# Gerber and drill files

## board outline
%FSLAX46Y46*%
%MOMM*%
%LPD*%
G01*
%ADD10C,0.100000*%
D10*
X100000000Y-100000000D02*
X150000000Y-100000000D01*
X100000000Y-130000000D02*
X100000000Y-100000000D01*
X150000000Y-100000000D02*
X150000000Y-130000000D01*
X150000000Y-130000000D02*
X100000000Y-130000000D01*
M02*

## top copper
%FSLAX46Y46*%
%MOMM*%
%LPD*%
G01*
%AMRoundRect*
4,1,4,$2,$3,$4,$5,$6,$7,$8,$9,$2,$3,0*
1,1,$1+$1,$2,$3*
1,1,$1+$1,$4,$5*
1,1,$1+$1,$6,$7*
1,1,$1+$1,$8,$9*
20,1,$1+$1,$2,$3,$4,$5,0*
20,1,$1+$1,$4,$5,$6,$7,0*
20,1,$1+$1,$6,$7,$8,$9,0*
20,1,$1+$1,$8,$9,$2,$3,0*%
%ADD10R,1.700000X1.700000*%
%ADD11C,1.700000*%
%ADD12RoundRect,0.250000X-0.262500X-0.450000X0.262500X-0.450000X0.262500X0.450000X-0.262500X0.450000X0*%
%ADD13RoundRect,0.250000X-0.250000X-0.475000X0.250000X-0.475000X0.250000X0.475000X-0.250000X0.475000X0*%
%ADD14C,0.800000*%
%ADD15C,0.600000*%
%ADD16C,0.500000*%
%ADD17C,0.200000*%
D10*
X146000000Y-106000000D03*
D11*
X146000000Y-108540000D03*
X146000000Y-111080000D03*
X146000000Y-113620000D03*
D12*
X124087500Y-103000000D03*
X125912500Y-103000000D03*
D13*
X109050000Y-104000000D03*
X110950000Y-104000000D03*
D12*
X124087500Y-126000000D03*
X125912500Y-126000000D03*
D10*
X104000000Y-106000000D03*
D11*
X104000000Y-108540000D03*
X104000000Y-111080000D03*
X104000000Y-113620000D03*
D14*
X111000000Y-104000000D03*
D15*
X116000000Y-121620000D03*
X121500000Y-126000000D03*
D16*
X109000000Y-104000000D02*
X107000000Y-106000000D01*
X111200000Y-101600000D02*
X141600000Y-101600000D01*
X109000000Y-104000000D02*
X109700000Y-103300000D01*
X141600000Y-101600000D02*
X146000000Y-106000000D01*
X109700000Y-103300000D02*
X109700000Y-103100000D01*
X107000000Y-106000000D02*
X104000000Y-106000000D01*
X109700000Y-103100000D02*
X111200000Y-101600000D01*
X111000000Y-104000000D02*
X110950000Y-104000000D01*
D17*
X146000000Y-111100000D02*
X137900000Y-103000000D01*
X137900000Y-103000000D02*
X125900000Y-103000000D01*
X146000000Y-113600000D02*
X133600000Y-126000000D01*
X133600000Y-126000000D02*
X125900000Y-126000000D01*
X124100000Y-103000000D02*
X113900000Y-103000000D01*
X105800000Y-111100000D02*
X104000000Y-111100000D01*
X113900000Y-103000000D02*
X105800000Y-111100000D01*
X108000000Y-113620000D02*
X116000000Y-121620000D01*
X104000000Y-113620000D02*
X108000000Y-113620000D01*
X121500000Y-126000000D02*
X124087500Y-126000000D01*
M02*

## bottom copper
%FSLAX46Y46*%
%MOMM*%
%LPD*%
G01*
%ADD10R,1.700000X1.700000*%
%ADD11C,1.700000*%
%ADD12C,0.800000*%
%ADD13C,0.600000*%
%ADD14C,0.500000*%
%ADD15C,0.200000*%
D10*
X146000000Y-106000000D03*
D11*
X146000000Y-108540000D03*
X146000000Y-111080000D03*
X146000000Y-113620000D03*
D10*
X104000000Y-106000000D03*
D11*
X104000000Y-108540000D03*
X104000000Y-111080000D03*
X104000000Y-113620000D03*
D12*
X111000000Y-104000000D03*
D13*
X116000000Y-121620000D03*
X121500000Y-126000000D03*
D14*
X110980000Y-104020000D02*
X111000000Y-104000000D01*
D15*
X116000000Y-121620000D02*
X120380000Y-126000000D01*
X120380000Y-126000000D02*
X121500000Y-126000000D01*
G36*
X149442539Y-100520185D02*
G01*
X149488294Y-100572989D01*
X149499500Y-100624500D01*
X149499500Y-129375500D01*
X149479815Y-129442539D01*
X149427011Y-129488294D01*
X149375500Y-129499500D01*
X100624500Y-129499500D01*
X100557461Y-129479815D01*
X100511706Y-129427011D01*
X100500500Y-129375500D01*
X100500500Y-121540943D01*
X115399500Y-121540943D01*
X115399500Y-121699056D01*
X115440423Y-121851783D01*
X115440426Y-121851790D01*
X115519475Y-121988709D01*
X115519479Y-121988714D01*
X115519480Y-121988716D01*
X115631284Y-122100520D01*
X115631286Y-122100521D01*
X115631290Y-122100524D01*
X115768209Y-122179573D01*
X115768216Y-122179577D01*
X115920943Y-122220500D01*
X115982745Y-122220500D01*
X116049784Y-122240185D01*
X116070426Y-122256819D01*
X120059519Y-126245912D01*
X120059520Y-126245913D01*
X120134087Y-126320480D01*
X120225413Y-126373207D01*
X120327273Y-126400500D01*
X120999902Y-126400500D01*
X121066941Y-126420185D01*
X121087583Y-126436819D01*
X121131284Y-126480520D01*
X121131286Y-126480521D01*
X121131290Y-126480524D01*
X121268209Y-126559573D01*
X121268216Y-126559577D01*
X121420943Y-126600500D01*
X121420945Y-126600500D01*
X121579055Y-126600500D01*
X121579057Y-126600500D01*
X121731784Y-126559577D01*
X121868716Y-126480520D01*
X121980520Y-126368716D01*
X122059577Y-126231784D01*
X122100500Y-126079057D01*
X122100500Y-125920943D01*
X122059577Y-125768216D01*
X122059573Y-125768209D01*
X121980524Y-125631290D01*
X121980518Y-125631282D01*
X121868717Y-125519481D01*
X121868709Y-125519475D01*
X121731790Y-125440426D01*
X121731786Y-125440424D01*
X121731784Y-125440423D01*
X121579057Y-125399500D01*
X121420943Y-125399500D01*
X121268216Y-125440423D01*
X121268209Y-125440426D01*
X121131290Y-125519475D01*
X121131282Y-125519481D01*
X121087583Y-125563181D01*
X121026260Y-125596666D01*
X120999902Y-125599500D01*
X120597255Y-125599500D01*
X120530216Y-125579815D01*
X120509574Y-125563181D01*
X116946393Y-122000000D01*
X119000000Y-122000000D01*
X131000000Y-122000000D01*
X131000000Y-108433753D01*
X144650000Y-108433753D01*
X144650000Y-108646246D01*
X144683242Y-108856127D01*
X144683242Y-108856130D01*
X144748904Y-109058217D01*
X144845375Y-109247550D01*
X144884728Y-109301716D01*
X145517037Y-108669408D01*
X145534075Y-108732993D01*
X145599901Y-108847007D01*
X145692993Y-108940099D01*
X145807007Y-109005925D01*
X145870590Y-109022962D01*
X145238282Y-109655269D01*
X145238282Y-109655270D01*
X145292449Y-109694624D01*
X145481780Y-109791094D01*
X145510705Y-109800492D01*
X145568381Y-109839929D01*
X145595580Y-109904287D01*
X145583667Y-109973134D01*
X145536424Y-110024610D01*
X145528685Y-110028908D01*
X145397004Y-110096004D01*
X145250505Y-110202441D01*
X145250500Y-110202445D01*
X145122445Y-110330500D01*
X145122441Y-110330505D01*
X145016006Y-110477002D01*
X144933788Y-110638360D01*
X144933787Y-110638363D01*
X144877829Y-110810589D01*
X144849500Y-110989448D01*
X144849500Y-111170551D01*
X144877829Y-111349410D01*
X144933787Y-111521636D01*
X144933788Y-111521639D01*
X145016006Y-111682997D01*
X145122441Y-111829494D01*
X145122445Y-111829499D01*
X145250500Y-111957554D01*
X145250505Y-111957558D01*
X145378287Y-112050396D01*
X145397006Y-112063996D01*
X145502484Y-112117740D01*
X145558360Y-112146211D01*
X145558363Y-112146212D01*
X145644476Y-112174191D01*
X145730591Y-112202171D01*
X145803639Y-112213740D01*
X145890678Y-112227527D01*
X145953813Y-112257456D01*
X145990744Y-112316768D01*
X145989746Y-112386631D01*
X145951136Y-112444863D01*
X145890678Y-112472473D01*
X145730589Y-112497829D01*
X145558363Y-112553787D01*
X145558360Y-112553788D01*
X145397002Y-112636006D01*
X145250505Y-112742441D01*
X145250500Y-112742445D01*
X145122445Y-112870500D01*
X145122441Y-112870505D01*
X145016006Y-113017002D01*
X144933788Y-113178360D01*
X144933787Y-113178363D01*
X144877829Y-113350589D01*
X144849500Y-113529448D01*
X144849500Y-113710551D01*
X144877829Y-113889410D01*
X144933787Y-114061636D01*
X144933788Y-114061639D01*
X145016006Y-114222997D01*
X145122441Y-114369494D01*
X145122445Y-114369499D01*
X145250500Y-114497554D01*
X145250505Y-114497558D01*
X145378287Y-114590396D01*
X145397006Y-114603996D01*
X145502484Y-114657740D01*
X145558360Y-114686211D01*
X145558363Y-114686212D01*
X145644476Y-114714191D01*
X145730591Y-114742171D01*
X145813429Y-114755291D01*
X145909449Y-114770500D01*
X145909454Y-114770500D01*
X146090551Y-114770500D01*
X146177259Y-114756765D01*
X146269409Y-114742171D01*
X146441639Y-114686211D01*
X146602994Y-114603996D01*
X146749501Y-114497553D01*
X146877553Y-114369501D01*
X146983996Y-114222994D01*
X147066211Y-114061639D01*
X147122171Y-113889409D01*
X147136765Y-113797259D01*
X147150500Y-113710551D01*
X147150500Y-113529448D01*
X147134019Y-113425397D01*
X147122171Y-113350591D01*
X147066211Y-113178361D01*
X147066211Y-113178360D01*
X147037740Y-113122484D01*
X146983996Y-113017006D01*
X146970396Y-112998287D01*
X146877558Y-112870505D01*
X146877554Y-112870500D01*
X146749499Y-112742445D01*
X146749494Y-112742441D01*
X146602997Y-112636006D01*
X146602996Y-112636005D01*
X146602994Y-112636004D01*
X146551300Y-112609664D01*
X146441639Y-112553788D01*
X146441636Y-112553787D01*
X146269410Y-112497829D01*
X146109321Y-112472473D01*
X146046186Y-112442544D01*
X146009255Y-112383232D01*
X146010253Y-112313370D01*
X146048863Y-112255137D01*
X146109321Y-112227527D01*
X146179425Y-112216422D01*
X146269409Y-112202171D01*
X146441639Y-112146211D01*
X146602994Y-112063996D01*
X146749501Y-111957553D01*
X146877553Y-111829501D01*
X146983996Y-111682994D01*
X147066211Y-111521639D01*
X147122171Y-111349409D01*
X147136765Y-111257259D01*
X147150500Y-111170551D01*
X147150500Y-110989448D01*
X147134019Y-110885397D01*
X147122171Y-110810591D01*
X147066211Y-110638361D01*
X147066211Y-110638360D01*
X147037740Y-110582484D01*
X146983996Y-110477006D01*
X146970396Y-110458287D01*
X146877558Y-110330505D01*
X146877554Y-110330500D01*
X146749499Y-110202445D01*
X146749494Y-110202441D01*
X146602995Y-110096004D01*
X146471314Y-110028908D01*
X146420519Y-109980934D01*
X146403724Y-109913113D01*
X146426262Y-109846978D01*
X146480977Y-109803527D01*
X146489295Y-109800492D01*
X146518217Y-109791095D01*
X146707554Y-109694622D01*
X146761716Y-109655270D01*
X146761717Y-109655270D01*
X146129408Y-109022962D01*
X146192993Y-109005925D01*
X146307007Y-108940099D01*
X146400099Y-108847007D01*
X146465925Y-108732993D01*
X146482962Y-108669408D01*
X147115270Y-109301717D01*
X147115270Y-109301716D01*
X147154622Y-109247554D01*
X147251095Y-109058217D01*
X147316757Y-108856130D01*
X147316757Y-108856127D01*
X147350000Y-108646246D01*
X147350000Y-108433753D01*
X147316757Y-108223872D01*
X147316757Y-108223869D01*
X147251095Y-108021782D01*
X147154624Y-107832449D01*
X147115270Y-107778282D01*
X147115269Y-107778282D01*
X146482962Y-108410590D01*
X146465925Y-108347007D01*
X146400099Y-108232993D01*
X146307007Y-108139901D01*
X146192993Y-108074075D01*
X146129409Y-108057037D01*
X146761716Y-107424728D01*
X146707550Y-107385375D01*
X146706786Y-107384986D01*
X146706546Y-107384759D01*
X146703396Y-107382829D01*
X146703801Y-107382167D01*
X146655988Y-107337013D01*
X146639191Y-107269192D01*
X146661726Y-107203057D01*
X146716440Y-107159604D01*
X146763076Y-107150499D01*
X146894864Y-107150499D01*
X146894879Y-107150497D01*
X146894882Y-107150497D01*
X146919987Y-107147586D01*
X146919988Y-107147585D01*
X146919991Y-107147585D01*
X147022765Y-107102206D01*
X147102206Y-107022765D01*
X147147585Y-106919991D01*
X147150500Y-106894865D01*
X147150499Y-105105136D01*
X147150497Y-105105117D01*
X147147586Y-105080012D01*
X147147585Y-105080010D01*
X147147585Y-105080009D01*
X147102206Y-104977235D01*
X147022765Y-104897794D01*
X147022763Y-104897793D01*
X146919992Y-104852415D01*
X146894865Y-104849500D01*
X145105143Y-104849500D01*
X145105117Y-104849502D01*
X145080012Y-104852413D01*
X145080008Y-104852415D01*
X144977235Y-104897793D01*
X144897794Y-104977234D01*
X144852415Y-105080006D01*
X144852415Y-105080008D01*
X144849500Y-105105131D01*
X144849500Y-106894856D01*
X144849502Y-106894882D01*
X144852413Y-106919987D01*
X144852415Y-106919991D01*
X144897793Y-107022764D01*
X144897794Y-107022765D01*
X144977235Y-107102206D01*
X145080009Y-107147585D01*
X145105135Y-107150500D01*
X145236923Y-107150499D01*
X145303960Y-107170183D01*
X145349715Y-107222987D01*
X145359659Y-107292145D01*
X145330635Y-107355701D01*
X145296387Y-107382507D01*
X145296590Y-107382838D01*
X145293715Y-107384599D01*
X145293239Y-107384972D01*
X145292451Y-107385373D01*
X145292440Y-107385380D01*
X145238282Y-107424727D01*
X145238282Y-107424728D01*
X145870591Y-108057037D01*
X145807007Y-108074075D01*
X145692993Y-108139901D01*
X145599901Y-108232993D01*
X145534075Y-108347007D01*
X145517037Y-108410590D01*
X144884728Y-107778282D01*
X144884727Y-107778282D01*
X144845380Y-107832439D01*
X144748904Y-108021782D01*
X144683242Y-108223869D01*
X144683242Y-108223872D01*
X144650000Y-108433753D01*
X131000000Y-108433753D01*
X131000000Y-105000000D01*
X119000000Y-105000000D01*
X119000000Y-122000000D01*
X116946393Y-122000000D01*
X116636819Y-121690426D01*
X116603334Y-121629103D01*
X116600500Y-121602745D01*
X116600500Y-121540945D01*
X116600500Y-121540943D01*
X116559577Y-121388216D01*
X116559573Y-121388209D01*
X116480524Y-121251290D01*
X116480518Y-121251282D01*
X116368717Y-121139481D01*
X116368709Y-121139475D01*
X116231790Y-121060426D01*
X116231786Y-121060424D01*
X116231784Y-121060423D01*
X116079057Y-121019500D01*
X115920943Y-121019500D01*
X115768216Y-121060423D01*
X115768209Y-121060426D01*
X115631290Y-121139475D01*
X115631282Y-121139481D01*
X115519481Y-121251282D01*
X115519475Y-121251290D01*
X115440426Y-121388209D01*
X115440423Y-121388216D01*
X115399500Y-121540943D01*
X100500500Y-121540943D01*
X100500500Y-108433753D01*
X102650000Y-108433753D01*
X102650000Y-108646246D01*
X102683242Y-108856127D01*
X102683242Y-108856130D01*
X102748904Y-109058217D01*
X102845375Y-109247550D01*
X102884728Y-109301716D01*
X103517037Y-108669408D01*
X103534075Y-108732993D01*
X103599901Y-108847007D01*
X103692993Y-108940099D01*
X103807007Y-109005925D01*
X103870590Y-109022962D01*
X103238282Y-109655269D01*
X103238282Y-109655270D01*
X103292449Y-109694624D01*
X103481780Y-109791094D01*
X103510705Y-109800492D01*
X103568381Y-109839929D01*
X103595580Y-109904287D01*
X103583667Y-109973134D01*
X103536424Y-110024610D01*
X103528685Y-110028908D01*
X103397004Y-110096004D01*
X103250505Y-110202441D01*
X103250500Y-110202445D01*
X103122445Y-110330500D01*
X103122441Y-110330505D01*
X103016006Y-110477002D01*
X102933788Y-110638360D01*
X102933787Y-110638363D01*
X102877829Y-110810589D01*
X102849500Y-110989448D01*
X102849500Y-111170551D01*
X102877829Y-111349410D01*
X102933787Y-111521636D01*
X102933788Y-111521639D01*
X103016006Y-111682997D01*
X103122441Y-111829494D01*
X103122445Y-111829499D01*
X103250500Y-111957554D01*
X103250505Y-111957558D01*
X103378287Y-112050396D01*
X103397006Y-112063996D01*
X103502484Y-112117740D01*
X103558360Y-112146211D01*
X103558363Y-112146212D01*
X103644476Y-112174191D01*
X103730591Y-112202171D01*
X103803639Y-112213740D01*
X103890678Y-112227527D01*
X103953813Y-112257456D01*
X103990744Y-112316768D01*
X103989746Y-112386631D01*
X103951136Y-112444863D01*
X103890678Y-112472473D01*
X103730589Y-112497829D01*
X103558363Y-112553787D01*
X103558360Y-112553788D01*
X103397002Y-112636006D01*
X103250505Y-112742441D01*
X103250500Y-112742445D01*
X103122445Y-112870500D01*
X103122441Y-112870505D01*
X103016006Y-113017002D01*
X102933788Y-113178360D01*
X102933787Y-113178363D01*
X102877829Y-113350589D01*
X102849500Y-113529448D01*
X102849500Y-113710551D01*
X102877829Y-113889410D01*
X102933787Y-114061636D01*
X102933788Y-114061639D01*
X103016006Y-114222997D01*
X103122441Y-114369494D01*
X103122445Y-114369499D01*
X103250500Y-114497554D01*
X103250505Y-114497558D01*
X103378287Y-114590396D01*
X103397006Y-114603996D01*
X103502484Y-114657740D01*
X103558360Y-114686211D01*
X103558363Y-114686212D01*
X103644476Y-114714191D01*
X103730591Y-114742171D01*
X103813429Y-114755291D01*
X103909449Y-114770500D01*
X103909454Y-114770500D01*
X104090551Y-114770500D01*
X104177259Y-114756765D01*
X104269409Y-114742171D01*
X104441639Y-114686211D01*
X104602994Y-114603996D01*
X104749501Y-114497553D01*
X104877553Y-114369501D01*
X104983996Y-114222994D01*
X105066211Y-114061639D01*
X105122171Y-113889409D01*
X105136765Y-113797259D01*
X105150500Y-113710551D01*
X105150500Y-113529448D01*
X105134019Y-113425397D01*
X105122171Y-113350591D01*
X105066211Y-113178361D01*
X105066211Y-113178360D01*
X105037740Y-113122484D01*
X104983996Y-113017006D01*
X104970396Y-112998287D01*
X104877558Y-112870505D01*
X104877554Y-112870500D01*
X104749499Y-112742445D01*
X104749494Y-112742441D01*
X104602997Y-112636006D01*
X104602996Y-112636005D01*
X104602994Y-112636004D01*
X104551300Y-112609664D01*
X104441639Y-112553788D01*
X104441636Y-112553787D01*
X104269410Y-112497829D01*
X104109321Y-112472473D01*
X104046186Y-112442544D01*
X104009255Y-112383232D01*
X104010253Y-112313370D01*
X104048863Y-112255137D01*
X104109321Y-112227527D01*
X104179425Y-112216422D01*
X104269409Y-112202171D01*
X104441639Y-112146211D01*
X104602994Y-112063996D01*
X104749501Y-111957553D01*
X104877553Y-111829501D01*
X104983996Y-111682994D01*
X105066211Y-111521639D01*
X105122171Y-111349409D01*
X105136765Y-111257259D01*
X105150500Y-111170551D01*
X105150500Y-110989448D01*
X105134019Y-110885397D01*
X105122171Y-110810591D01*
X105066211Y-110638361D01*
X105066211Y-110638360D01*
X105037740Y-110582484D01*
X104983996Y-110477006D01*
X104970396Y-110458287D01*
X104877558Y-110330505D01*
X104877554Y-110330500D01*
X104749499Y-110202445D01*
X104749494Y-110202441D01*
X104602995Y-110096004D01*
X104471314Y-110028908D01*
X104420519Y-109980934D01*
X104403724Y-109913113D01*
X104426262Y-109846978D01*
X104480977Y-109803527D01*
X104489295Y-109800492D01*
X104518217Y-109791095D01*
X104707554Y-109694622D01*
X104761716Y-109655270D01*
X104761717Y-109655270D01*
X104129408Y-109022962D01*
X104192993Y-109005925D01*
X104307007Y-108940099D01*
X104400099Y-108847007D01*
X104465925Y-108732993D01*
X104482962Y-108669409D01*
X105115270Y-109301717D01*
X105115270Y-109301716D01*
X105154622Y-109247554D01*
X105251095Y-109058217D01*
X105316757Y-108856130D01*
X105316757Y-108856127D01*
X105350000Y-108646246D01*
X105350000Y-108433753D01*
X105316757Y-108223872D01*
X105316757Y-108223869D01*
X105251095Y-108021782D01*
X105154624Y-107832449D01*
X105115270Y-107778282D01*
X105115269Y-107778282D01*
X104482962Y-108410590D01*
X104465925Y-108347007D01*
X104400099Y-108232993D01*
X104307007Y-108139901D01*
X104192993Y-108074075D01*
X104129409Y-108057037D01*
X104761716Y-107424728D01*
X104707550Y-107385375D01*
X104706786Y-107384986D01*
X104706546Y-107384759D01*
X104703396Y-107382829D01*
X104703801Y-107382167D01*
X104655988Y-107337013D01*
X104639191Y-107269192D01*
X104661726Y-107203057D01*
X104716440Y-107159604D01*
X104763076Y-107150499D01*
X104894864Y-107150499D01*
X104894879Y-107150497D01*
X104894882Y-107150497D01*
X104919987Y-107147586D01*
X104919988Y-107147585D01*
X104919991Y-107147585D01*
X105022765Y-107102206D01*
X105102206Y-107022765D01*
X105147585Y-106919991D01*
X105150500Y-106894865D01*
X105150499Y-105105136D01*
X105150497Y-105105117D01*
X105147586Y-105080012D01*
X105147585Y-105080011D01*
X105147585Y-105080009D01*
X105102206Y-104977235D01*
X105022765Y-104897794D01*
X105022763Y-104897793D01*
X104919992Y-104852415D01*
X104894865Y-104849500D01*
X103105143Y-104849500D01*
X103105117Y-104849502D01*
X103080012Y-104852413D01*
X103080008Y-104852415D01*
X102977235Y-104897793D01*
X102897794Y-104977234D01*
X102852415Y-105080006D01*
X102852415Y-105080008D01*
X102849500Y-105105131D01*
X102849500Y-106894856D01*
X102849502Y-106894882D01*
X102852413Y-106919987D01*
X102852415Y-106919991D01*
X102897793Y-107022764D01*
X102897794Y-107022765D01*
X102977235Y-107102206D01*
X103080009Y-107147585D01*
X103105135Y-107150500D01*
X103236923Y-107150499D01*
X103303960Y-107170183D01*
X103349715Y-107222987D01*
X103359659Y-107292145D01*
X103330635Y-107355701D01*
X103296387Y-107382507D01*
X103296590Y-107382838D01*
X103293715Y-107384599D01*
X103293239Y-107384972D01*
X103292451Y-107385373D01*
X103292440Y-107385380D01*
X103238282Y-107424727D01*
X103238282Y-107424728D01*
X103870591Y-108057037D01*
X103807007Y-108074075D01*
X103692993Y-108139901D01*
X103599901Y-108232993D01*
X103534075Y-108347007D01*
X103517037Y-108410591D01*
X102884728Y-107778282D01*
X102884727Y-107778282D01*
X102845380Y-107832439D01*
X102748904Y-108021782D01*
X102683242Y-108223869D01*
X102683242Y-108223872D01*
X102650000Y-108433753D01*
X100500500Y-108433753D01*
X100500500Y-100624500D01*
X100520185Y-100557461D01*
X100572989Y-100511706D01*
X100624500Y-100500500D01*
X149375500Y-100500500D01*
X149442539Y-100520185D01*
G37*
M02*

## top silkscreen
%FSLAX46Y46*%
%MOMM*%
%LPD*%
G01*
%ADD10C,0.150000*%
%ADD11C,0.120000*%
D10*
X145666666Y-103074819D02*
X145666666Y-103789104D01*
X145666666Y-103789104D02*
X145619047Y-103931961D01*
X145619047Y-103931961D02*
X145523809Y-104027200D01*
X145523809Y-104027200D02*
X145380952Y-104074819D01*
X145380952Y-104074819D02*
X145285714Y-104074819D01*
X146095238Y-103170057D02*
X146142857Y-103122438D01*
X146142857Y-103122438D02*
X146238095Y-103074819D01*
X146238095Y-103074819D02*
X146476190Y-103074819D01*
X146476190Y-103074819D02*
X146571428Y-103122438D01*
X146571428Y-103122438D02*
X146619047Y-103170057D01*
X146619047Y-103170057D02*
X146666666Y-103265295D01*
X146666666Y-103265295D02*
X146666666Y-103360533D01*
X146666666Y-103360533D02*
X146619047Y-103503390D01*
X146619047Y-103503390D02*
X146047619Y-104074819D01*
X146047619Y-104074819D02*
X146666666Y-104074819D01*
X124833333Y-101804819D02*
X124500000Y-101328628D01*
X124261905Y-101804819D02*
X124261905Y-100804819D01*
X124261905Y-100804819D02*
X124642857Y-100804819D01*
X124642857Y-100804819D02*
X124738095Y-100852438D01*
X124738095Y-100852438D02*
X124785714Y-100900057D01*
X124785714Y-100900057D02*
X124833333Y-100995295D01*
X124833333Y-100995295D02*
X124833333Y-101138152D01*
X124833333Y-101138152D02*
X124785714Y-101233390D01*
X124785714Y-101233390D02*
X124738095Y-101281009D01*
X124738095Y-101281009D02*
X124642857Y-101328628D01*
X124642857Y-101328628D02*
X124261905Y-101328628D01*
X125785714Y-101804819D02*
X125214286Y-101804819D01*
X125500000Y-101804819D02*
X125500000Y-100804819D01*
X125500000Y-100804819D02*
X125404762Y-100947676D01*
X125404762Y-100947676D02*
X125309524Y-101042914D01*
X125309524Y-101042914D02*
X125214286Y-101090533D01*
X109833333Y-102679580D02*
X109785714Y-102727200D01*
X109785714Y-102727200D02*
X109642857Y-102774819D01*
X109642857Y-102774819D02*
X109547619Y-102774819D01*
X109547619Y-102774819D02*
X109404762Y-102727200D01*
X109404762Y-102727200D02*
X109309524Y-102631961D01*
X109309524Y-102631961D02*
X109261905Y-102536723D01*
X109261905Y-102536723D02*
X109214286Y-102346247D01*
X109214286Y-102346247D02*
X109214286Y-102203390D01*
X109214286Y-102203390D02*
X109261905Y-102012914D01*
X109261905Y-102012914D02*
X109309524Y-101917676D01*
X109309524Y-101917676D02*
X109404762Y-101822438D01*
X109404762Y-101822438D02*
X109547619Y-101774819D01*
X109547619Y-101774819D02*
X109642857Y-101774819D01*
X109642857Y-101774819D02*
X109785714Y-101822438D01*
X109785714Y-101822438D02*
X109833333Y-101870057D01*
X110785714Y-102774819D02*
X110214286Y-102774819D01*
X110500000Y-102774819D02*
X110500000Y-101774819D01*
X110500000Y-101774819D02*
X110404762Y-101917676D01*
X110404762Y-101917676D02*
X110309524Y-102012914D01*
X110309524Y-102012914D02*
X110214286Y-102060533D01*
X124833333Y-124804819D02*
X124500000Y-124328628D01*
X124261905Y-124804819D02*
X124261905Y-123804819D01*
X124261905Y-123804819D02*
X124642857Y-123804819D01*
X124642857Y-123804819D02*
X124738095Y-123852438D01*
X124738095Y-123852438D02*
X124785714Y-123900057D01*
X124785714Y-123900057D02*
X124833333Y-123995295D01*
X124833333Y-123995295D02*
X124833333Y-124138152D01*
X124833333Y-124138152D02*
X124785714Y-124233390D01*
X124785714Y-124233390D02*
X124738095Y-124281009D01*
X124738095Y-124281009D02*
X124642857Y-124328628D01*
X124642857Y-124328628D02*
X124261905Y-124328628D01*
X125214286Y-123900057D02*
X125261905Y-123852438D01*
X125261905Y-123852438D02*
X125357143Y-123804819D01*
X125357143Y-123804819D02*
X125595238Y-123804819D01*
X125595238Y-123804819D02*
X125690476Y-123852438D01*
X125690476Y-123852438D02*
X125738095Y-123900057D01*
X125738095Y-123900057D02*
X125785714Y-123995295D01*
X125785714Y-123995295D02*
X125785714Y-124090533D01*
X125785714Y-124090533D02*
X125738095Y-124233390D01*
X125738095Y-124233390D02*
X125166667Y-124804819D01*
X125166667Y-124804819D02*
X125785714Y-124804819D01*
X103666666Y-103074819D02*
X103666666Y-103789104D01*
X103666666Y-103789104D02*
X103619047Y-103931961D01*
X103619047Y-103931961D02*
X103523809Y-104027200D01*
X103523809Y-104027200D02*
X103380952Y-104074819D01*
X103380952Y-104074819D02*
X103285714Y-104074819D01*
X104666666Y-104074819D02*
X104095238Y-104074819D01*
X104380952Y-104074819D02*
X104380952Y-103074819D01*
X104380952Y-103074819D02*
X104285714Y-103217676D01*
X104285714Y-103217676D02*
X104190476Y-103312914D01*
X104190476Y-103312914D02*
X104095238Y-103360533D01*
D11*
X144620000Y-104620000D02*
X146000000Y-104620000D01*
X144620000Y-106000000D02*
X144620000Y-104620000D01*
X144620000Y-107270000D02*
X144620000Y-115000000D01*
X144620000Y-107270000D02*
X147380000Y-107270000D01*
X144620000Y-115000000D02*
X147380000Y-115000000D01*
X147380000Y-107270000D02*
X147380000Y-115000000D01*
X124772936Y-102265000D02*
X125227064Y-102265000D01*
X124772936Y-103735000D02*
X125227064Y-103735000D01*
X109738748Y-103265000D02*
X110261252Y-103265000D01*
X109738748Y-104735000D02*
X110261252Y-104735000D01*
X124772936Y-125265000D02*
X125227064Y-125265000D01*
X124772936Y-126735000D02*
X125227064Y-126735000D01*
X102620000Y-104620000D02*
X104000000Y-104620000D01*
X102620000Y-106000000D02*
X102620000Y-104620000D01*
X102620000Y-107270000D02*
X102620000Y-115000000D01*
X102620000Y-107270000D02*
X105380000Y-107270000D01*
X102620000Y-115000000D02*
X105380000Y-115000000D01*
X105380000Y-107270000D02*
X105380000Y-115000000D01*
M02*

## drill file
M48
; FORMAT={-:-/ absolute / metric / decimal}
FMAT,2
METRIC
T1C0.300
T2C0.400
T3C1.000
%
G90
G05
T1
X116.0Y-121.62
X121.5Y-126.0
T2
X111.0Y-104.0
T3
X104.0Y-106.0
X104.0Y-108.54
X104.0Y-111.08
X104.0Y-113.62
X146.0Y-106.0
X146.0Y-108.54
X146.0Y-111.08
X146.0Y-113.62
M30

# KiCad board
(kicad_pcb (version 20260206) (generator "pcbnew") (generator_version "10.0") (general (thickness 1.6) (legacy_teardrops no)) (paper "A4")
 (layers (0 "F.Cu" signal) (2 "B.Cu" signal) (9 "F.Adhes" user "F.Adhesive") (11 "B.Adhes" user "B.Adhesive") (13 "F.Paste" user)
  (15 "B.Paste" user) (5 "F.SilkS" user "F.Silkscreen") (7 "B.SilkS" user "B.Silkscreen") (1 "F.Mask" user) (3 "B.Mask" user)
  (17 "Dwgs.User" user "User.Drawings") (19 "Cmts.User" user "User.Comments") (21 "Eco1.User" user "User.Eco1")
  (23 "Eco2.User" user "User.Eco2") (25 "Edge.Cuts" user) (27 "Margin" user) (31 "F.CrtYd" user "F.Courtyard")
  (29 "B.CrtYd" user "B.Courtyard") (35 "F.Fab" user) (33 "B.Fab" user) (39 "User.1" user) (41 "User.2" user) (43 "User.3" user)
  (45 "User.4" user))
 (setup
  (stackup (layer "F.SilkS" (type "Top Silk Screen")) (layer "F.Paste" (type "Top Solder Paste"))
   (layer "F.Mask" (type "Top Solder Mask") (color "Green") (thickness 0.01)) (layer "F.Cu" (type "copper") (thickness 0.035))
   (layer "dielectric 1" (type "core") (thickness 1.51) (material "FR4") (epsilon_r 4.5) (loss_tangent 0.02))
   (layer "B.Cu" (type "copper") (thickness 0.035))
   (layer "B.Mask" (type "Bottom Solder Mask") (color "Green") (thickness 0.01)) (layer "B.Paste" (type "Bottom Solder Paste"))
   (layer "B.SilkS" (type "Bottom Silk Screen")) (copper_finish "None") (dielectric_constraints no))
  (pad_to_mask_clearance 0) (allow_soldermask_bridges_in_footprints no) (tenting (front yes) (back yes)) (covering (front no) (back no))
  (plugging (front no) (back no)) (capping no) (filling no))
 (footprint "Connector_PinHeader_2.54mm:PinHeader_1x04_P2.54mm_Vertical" (layer "F.Cu") (at 146 106)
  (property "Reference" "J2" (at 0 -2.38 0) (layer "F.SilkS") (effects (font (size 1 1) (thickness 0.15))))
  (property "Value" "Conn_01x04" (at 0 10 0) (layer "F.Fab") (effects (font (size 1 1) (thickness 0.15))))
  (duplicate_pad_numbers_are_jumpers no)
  (fp_line (start -1.38 -1.38) (end 0 -1.38) (stroke (width 0.12) (type solid)) (layer "F.SilkS"))
  (fp_line (start -1.38 0) (end -1.38 -1.38) (stroke (width 0.12) (type solid)) (layer "F.SilkS"))
  (fp_line (start -1.38 1.27) (end -1.38 9) (stroke (width 0.12) (type solid)) (layer "F.SilkS"))
  (fp_line (start -1.38 1.27) (end 1.38 1.27) (stroke (width 0.12) (type solid)) (layer "F.SilkS"))
  (fp_line (start -1.38 9) (end 1.38 9) (stroke (width 0.12) (type solid)) (layer "F.SilkS"))
  (fp_line (start 1.38 1.27) (end 1.38 9) (stroke (width 0.12) (type solid)) (layer "F.SilkS"))
  (pad "1" thru_hole rect (at 0 0) (size 1.7 1.7) (drill 1) (layers "*.Cu" "*.Mask") (remove_unused_layers no) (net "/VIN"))
  (pad "2" thru_hole circle (at 0 2.54) (size 1.7 1.7) (drill 1) (layers "*.Cu" "*.Mask") (remove_unused_layers no) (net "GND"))
  (pad "3" thru_hole circle (at 0 5.08) (size 1.7 1.7) (drill 1) (layers "*.Cu" "*.Mask") (remove_unused_layers no) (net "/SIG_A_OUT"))
  (pad "4" thru_hole circle (at 0 7.62) (size 1.7 1.7) (drill 1) (layers "*.Cu" "*.Mask") (remove_unused_layers no) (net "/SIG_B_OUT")))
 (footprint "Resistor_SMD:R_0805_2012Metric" (layer "F.Cu") (at 125 103)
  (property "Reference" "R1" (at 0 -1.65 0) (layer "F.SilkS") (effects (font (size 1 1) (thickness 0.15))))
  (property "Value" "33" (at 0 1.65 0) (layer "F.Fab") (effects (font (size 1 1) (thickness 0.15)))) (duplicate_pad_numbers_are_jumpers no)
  (fp_line (start -0.227064 -0.735) (end 0.227064 -0.735) (stroke (width 0.12) (type solid)) (layer "F.SilkS"))
  (fp_line (start -0.227064 0.735) (end 0.227064 0.735) (stroke (width 0.12) (type solid)) (layer "F.SilkS"))
  (pad "1" smd roundrect (at -0.9125 0) (size 1.025 1.4) (layers "F.Cu" "F.Mask" "F.Paste") (roundrect_rratio 0.243902) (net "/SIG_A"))
  (pad "2" smd roundrect (at 0.9125 0) (size 1.025 1.4) (layers "F.Cu" "F.Mask" "F.Paste") (roundrect_rratio 0.243902) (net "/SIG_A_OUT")))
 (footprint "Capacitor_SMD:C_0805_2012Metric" (layer "F.Cu") (at 110 104)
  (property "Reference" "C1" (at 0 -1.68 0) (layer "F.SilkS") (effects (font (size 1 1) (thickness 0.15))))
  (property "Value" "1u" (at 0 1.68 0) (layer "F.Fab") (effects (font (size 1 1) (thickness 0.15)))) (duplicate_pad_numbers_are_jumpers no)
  (fp_line (start -0.261252 -0.735) (end 0.261252 -0.735) (stroke (width 0.12) (type solid)) (layer "F.SilkS"))
  (fp_line (start -0.261252 0.735) (end 0.261252 0.735) (stroke (width 0.12) (type solid)) (layer "F.SilkS"))
  (pad "1" smd roundrect (at -0.95 0) (size 1 1.45) (layers "F.Cu" "F.Mask" "F.Paste") (roundrect_rratio 0.25) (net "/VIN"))
  (pad "2" smd roundrect (at 0.95 0) (size 1 1.45) (layers "F.Cu" "F.Mask" "F.Paste") (roundrect_rratio 0.25) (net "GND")))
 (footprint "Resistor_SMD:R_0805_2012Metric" (layer "F.Cu") (at 125 126)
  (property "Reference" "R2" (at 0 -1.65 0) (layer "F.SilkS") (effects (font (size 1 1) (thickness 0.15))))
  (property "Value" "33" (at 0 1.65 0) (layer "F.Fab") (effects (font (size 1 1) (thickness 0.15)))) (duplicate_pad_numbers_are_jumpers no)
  (fp_line (start -0.227064 -0.735) (end 0.227064 -0.735) (stroke (width 0.12) (type solid)) (layer "F.SilkS"))
  (fp_line (start -0.227064 0.735) (end 0.227064 0.735) (stroke (width 0.12) (type solid)) (layer "F.SilkS"))
  (pad "1" smd roundrect (at -0.9125 0) (size 1.025 1.4) (layers "F.Cu" "F.Mask" "F.Paste") (roundrect_rratio 0.243902) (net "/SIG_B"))
  (pad "2" smd roundrect (at 0.9125 0) (size 1.025 1.4) (layers "F.Cu" "F.Mask" "F.Paste") (roundrect_rratio 0.243902) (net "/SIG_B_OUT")))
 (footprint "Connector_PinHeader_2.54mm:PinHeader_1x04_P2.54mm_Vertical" (layer "F.Cu") (at 104 106)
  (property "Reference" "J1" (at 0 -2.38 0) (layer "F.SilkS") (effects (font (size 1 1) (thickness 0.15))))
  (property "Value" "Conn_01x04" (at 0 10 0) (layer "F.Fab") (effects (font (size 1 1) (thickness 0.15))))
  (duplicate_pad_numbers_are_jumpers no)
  (fp_line (start -1.38 -1.38) (end 0 -1.38) (stroke (width 0.12) (type solid)) (layer "F.SilkS"))
  (fp_line (start -1.38 0) (end -1.38 -1.38) (stroke (width 0.12) (type solid)) (layer "F.SilkS"))
  (fp_line (start -1.38 1.27) (end -1.38 9) (stroke (width 0.12) (type solid)) (layer "F.SilkS"))
  (fp_line (start -1.38 1.27) (end 1.38 1.27) (stroke (width 0.12) (type solid)) (layer "F.SilkS"))
  (fp_line (start -1.38 9) (end 1.38 9) (stroke (width 0.12) (type solid)) (layer "F.SilkS"))
  (fp_line (start 1.38 1.27) (end 1.38 9) (stroke (width 0.12) (type solid)) (layer "F.SilkS"))
  (pad "1" thru_hole rect (at 0 0) (size 1.7 1.7) (drill 1) (layers "*.Cu" "*.Mask") (remove_unused_layers no) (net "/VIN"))
  (pad "2" thru_hole circle (at 0 2.54) (size 1.7 1.7) (drill 1) (layers "*.Cu" "*.Mask") (remove_unused_layers no) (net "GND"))
  (pad "3" thru_hole circle (at 0 5.08) (size 1.7 1.7) (drill 1) (layers "*.Cu" "*.Mask") (remove_unused_layers no) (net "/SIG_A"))
  (pad "4" thru_hole circle (at 0 7.62) (size 1.7 1.7) (drill 1) (layers "*.Cu" "*.Mask") (remove_unused_layers no) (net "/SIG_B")))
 (gr_line (start 100 100) (end 150 100) (stroke (width 0.1) (type default)) (layer "Edge.Cuts"))
 (gr_line (start 100 130) (end 100 100) (stroke (width 0.1) (type default)) (layer "Edge.Cuts"))
 (gr_line (start 150 100) (end 150 130) (stroke (width 0.1) (type default)) (layer "Edge.Cuts"))
 (gr_line (start 150 130) (end 100 130) (stroke (width 0.1) (type default)) (layer "Edge.Cuts"))
 (segment (start 109 104) (end 107 106) (width 0.5) (layer "F.Cu") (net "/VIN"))
 (segment (start 111.2 101.6) (end 141.6 101.6) (width 0.5) (layer "F.Cu") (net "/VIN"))
 (segment (start 109 104) (end 109.7 103.3) (width 0.5) (layer "F.Cu") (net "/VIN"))
 (segment (start 141.6 101.6) (end 146 106) (width 0.5) (layer "F.Cu") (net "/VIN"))
 (segment (start 109.7 103.3) (end 109.7 103.1) (width 0.5) (layer "F.Cu") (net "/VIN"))
 (segment (start 107 106) (end 104 106) (width 0.5) (layer "F.Cu") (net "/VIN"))
 (segment (start 109.7 103.1) (end 111.2 101.6) (width 0.5) (layer "F.Cu") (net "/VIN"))
 (segment (start 111 104) (end 110.95 104) (width 0.5) (layer "F.Cu") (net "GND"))
 (via (at 111 104) (size 0.8) (drill 0.4) (layers "F.Cu" "B.Cu") (capping yes) (filling yes) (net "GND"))
 (segment (start 110.98 104.02) (end 111 104) (width 0.5) (layer "B.Cu") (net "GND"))
 (segment (start 146 111.1) (end 137.9 103) (width 0.2) (layer "F.Cu") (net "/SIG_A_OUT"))
 (segment (start 137.9 103) (end 125.9 103) (width 0.2) (layer "F.Cu") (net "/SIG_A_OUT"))
 (segment (start 146 113.6) (end 133.6 126) (width 0.2) (layer "F.Cu") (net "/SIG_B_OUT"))
 (segment (start 133.6 126) (end 125.9 126) (width 0.2) (layer "F.Cu") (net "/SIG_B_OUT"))
 (segment (start 124.1 103) (end 113.9 103) (width 0.2) (layer "F.Cu") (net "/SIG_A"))
 (segment (start 105.8 111.1) (end 104 111.1) (width 0.2) (layer "F.Cu") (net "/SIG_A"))
 (segment (start 113.9 103) (end 105.8 111.1) (width 0.2) (layer "F.Cu") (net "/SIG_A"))
 (segment (start 108 113.62) (end 116 121.62) (width 0.2) (locked yes) (layer "F.Cu") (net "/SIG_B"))
 (segment (start 104 113.62) (end 108 113.62) (width 0.2) (locked yes) (layer "F.Cu") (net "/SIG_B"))
 (segment (start 121.5 126) (end 124.0875 126) (width 0.2) (locked yes) (layer "F.Cu") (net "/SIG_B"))
 (via (at 116 121.62) (size 0.6) (drill 0.3) (layers "F.Cu" "B.Cu") (locked yes) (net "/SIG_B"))
 (via (at 121.5 126) (size 0.6) (drill 0.3) (layers "F.Cu" "B.Cu") (locked yes) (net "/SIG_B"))
 (segment (start 116 121.62) (end 120.38 126) (width 0.2) (locked yes) (layer "B.Cu") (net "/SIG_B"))
 (segment (start 120.38 126) (end 121.5 126) (width 0.2) (locked yes) (layer "B.Cu") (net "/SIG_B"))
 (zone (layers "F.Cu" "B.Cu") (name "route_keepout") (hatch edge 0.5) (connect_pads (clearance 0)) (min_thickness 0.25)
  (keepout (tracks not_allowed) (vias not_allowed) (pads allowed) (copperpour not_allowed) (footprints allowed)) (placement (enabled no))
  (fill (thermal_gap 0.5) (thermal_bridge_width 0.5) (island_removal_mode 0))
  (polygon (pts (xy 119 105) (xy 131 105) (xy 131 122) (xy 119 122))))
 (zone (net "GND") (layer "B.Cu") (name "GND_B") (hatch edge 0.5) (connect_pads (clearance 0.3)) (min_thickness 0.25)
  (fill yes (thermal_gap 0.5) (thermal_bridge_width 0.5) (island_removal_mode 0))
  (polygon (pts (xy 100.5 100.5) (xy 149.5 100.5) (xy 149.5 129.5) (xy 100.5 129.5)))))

